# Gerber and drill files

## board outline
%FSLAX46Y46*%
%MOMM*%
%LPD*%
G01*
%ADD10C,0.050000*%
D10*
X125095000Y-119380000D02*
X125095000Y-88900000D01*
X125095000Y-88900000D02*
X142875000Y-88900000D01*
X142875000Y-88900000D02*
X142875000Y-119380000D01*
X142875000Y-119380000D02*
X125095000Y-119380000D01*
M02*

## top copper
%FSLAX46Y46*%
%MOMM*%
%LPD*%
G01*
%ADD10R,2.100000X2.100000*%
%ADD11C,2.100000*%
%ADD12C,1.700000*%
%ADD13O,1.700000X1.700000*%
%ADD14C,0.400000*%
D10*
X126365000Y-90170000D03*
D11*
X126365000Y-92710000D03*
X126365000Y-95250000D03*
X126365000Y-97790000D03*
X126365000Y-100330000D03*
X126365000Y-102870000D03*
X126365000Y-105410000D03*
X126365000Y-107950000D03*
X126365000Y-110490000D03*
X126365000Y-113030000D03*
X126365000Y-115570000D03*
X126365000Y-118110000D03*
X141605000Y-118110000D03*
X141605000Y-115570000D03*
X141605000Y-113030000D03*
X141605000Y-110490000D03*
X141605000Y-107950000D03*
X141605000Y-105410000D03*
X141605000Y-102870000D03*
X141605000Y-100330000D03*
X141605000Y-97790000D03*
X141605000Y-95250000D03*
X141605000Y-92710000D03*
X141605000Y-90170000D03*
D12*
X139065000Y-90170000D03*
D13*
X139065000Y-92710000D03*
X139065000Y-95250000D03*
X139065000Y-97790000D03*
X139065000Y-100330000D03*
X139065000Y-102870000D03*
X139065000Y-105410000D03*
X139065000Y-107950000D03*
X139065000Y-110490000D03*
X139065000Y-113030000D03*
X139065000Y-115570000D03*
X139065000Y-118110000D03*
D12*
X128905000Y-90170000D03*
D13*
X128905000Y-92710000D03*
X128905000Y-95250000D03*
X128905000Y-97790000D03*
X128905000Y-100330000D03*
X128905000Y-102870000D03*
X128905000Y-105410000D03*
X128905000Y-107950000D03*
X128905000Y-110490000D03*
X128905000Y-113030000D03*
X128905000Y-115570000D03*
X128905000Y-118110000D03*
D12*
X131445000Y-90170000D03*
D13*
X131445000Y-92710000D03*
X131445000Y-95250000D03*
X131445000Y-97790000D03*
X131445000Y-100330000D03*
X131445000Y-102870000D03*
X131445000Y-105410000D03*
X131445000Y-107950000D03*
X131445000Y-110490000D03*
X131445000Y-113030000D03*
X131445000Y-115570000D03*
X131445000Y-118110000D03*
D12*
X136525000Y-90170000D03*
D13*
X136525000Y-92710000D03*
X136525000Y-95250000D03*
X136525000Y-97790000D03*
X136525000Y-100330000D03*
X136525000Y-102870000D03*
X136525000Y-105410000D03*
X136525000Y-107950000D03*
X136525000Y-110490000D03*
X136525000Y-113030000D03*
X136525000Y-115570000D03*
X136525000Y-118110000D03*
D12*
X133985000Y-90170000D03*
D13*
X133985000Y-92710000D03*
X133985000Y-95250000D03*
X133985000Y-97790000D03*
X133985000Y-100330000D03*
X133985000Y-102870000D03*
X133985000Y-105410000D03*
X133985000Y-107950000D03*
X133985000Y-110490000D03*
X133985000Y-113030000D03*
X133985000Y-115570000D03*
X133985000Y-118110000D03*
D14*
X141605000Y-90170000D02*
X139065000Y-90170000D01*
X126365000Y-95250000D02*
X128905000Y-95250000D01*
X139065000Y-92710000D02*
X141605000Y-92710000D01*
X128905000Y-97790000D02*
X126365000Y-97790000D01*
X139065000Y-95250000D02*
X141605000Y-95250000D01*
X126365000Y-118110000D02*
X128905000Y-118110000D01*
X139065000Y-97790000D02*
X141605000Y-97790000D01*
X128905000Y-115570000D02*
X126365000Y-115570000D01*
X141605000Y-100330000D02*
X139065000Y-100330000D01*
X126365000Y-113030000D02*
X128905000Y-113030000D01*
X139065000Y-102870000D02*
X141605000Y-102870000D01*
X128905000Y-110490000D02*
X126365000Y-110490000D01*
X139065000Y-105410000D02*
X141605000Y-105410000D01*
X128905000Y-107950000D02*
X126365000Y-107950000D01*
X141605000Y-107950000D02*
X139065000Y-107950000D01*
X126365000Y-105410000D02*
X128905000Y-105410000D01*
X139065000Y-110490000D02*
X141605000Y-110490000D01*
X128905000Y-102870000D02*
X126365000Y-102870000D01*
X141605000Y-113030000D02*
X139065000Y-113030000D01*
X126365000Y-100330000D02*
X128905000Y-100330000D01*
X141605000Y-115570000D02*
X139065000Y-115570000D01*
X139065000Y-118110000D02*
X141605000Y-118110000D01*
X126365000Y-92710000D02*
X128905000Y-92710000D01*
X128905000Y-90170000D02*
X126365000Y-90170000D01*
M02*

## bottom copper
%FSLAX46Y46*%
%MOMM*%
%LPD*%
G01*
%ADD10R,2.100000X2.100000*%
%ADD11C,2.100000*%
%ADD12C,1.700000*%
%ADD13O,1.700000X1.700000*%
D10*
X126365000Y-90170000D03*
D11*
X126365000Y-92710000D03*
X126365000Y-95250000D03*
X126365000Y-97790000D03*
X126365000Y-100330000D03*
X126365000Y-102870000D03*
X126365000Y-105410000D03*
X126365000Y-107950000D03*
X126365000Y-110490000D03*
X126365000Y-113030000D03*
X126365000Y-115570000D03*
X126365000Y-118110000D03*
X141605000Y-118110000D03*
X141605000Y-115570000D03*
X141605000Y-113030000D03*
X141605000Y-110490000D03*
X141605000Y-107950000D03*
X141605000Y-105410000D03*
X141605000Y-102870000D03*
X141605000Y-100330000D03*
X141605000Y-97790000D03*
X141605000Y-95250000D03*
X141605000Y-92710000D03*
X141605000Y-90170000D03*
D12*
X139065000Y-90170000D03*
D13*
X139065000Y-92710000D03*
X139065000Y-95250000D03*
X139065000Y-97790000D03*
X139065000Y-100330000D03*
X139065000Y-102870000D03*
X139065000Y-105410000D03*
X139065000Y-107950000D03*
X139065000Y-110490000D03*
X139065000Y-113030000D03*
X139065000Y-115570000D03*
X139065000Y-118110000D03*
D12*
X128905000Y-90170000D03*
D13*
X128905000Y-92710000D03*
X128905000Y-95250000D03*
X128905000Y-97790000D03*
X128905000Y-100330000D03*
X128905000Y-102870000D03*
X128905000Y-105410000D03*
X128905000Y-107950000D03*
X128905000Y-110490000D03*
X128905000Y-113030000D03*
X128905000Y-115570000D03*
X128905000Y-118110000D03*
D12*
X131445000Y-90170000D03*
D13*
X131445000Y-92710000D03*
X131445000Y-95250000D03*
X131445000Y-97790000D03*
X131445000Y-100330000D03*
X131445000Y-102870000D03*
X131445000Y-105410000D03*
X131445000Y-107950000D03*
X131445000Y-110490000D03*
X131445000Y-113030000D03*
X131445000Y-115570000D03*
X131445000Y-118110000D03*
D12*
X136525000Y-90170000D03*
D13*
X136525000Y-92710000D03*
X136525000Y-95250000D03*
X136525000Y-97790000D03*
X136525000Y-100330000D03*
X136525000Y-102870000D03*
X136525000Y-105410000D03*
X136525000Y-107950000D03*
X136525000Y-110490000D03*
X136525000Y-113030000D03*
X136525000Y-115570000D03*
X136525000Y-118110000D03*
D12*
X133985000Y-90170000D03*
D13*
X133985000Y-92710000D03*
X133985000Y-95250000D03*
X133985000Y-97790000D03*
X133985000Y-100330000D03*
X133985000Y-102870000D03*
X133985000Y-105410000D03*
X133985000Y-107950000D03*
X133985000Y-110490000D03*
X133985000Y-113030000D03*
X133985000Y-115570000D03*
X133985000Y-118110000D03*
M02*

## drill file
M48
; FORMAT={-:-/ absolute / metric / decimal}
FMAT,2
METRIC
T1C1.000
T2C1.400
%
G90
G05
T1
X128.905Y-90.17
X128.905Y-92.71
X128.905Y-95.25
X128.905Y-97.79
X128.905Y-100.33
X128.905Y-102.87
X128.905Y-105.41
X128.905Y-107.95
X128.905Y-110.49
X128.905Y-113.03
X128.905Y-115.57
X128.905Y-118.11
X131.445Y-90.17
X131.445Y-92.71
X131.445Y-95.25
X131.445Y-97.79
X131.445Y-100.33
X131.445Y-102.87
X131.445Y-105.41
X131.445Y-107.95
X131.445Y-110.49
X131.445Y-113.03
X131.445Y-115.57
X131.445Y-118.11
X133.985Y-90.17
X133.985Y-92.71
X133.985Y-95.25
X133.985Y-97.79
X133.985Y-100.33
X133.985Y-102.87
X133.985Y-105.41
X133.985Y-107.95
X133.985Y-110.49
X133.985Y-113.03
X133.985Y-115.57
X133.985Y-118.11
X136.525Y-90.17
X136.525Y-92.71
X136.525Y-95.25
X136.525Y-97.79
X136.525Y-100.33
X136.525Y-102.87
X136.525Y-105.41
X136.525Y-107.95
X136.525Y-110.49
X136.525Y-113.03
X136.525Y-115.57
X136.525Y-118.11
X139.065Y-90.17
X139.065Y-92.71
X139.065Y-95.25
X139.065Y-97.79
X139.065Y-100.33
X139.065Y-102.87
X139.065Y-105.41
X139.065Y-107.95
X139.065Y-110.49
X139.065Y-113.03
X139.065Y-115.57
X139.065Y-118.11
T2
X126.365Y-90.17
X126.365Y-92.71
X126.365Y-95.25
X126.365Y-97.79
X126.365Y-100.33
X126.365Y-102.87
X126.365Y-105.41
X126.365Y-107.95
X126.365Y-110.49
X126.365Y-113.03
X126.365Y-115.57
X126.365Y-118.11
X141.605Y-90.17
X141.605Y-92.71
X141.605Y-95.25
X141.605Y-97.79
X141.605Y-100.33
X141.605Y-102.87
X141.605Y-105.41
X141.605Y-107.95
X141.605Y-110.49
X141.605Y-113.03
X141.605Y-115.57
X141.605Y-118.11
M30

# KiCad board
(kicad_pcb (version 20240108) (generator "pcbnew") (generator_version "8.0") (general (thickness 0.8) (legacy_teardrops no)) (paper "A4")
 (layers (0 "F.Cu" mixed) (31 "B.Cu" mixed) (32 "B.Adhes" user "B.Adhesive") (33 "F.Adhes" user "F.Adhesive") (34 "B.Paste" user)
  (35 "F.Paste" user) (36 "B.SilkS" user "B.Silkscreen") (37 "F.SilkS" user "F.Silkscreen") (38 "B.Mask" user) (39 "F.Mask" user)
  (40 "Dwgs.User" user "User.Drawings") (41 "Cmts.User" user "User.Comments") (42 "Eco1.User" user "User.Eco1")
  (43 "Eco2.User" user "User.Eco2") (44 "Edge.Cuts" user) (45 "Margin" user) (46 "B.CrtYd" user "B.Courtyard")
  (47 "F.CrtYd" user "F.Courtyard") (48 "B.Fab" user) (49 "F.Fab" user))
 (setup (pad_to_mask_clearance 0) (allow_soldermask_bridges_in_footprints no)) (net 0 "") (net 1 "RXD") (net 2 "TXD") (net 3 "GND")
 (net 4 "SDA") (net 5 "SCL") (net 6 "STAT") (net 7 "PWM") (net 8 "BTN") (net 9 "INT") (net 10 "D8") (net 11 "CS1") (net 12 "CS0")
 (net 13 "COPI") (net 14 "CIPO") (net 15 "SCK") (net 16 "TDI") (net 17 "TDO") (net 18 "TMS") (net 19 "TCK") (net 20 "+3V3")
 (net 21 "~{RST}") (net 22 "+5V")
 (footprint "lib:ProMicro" (layer "F.Cu") (at 126.365 90.17)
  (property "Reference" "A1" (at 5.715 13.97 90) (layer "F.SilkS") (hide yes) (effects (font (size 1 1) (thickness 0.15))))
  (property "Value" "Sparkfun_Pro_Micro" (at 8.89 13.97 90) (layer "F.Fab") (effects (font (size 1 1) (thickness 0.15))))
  (pad "1" thru_hole rect (at 0 0) (size 2.1 2.1) (drill 1.4) (layers "*.Cu" "*.Mask") (remove_unused_layers no) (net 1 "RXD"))
  (pad "2" thru_hole circle (at 0 2.54) (size 2.1 2.1) (drill 1.4) (layers "*.Cu" "*.Mask") (remove_unused_layers no) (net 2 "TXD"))
  (pad "3" thru_hole circle (at 0 5.08) (size 2.1 2.1) (drill 1.4) (layers "*.Cu" "*.Mask") (remove_unused_layers no) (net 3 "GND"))
  (pad "4" thru_hole circle (at 0 7.62) (size 2.1 2.1) (drill 1.4) (layers "*.Cu" "*.Mask") (remove_unused_layers no) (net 3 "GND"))
  (pad "5" thru_hole circle (at 0 10.16) (size 2.1 2.1) (drill 1.4) (layers "*.Cu" "*.Mask") (remove_unused_layers no) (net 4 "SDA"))
  (pad "6" thru_hole circle (at 0 12.7) (size 2.1 2.1) (drill 1.4) (layers "*.Cu" "*.Mask") (remove_unused_layers no) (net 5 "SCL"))
  (pad "7" thru_hole circle (at 0 15.24) (size 2.1 2.1) (drill 1.4) (layers "*.Cu" "*.Mask") (remove_unused_layers no) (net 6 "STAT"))
  (pad "8" thru_hole circle (at 0 17.78) (size 2.1 2.1) (drill 1.4) (layers "*.Cu" "*.Mask") (remove_unused_layers no) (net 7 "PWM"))
  (pad "9" thru_hole circle (at 0 20.32) (size 2.1 2.1) (drill 1.4) (layers "*.Cu" "*.Mask") (remove_unused_layers no) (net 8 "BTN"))
  (pad "10" thru_hole circle (at 0 22.86) (size 2.1 2.1) (drill 1.4) (layers "*.Cu" "*.Mask") (remove_unused_layers no) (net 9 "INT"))
  (pad "11" thru_hole circle (at 0 25.4) (size 2.1 2.1) (drill 1.4) (layers "*.Cu" "*.Mask") (remove_unused_layers no) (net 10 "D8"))
  (pad "12" thru_hole circle (at 0 27.94) (size 2.1 2.1) (drill 1.4) (layers "*.Cu" "*.Mask") (remove_unused_layers no) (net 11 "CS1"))
  (pad "13" thru_hole circle (at 15.24 27.94) (size 2.1 2.1) (drill 1.4) (layers "*.Cu" "*.Mask") (remove_unused_layers no) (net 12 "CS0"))
  (pad "14" thru_hole circle (at 15.24 25.4) (size 2.1 2.1) (drill 1.4) (layers "*.Cu" "*.Mask") (remove_unused_layers no) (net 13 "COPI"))
  (pad "15" thru_hole circle (at 15.24 22.86) (size 2.1 2.1) (drill 1.4) (layers "*.Cu" "*.Mask") (remove_unused_layers no) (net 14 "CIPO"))
  (pad "16" thru_hole circle (at 15.24 20.32) (size 2.1 2.1) (drill 1.4) (layers "*.Cu" "*.Mask") (remove_unused_layers no) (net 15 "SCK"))
  (pad "17" thru_hole circle (at 15.24 17.78) (size 2.1 2.1) (drill 1.4) (layers "*.Cu" "*.Mask") (remove_unused_layers no) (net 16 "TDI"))
  (pad "18" thru_hole circle (at 15.24 15.24) (size 2.1 2.1) (drill 1.4) (layers "*.Cu" "*.Mask") (remove_unused_layers no) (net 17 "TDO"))
  (pad "19" thru_hole circle (at 15.24 12.7) (size 2.1 2.1) (drill 1.4) (layers "*.Cu" "*.Mask") (remove_unused_layers no) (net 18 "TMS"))
  (pad "20" thru_hole circle (at 15.24 10.16) (size 2.1 2.1) (drill 1.4) (layers "*.Cu" "*.Mask") (remove_unused_layers no) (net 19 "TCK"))
  (pad "21" thru_hole circle (at 15.24 7.62) (size 2.1 2.1) (drill 1.4) (layers "*.Cu" "*.Mask") (remove_unused_layers no) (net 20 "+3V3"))
  (pad "22" thru_hole circle (at 15.24 5.08) (size 2.1 2.1) (drill 1.4) (layers "*.Cu" "*.Mask") (remove_unused_layers no) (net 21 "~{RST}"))
  (pad "23" thru_hole circle (at 15.24 2.54) (size 2.1 2.1) (drill 1.4) (layers "*.Cu" "*.Mask") (remove_unused_layers no) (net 3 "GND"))
  (pad "24" thru_hole circle (at 15.24 0) (size 2.1 2.1) (drill 1.4) (layers "*.Cu" "*.Mask") (remove_unused_layers no) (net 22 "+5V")))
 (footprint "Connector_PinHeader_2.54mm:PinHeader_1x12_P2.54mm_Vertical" (layer "F.Cu") (at 139.065 90.17)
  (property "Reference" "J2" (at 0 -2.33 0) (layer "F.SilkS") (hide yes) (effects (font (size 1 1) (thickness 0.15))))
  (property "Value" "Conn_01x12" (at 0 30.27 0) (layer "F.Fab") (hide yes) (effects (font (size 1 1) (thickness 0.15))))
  (pad "1" thru_hole circle (at 0 0) (size 1.7 1.7) (drill 1) (layers "*.Cu" "*.Mask") (remove_unused_layers no) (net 22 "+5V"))
  (pad "2" thru_hole oval (at 0 2.54) (size 1.7 1.7) (drill 1) (layers "*.Cu" "*.Mask") (remove_unused_layers no) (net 3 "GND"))
  (pad "3" thru_hole oval (at 0 5.08) (size 1.7 1.7) (drill 1) (layers "*.Cu" "*.Mask") (remove_unused_layers no) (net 21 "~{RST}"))
  (pad "4" thru_hole oval (at 0 7.62) (size 1.7 1.7) (drill 1) (layers "*.Cu" "*.Mask") (remove_unused_layers no) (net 20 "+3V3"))
  (pad "5" thru_hole oval (at 0 10.16) (size 1.7 1.7) (drill 1) (layers "*.Cu" "*.Mask") (remove_unused_layers no) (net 19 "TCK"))
  (pad "6" thru_hole oval (at 0 12.7) (size 1.7 1.7) (drill 1) (layers "*.Cu" "*.Mask") (remove_unused_layers no) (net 18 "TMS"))
  (pad "7" thru_hole oval (at 0 15.24) (size 1.7 1.7) (drill 1) (layers "*.Cu" "*.Mask") (remove_unused_layers no) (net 17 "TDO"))
  (pad "8" thru_hole oval (at 0 17.78) (size 1.7 1.7) (drill 1) (layers "*.Cu" "*.Mask") (remove_unused_layers no) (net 16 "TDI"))
  (pad "9" thru_hole oval (at 0 20.32) (size 1.7 1.7) (drill 1) (layers "*.Cu" "*.Mask") (remove_unused_layers no) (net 15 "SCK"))
  (pad "10" thru_hole oval (at 0 22.86) (size 1.7 1.7) (drill 1) (layers "*.Cu" "*.Mask") (remove_unused_layers no) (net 14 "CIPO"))
  (pad "11" thru_hole oval (at 0 25.4) (size 1.7 1.7) (drill 1) (layers "*.Cu" "*.Mask") (remove_unused_layers no) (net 13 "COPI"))
  (pad "12" thru_hole oval (at 0 27.94) (size 1.7 1.7) (drill 1) (layers "*.Cu" "*.Mask") (remove_unused_layers no) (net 12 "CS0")))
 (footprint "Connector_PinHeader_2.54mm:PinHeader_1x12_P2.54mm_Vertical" (layer "F.Cu") (at 128.905 90.17)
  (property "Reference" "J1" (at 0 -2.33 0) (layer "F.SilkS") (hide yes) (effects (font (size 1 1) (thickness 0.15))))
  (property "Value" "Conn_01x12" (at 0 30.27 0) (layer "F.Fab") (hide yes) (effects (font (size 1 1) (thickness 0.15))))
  (pad "1" thru_hole circle (at 0 0) (size 1.7 1.7) (drill 1) (layers "*.Cu" "*.Mask") (remove_unused_layers no) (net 1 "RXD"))
  (pad "2" thru_hole oval (at 0 2.54) (size 1.7 1.7) (drill 1) (layers "*.Cu" "*.Mask") (remove_unused_layers no) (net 2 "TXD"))
  (pad "3" thru_hole oval (at 0 5.08) (size 1.7 1.7) (drill 1) (layers "*.Cu" "*.Mask") (remove_unused_layers no) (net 3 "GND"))
  (pad "4" thru_hole oval (at 0 7.62) (size 1.7 1.7) (drill 1) (layers "*.Cu" "*.Mask") (remove_unused_layers no) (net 3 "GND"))
  (pad "5" thru_hole oval (at 0 10.16) (size 1.7 1.7) (drill 1) (layers "*.Cu" "*.Mask") (remove_unused_layers no) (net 4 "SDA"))
  (pad "6" thru_hole oval (at 0 12.7) (size 1.7 1.7) (drill 1) (layers "*.Cu" "*.Mask") (remove_unused_layers no) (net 5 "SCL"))
  (pad "7" thru_hole oval (at 0 15.24) (size 1.7 1.7) (drill 1) (layers "*.Cu" "*.Mask") (remove_unused_layers no) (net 6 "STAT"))
  (pad "8" thru_hole oval (at 0 17.78) (size 1.7 1.7) (drill 1) (layers "*.Cu" "*.Mask") (remove_unused_layers no) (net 7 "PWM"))
  (pad "9" thru_hole oval (at 0 20.32) (size 1.7 1.7) (drill 1) (layers "*.Cu" "*.Mask") (remove_unused_layers no) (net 8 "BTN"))
  (pad "10" thru_hole oval (at 0 22.86) (size 1.7 1.7) (drill 1) (layers "*.Cu" "*.Mask") (remove_unused_layers no) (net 9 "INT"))
  (pad "11" thru_hole oval (at 0 25.4) (size 1.7 1.7) (drill 1) (layers "*.Cu" "*.Mask") (remove_unused_layers no) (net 10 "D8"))
  (pad "12" thru_hole oval (at 0 27.94) (size 1.7 1.7) (drill 1) (layers "*.Cu" "*.Mask") (remove_unused_layers no) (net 11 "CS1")))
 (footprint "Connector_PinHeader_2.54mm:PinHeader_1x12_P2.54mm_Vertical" (layer "F.Cu") (at 131.445 90.17)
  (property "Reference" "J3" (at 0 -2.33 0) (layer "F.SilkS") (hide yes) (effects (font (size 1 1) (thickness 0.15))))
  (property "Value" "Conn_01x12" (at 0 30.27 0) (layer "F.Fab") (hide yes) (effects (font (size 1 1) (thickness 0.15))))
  (pad "1" thru_hole circle (at 0 0) (size 1.7 1.7) (drill 1) (layers "*.Cu" "*.Mask") (remove_unused_layers no))
  (pad "2" thru_hole oval (at 0 2.54) (size 1.7 1.7) (drill 1) (layers "*.Cu" "*.Mask") (remove_unused_layers no))
  (pad "3" thru_hole oval (at 0 5.08) (size 1.7 1.7) (drill 1) (layers "*.Cu" "*.Mask") (remove_unused_layers no))
  (pad "4" thru_hole oval (at 0 7.62) (size 1.7 1.7) (drill 1) (layers "*.Cu" "*.Mask") (remove_unused_layers no))
  (pad "5" thru_hole oval (at 0 10.16) (size 1.7 1.7) (drill 1) (layers "*.Cu" "*.Mask") (remove_unused_layers no))
  (pad "6" thru_hole oval (at 0 12.7) (size 1.7 1.7) (drill 1) (layers "*.Cu" "*.Mask") (remove_unused_layers no))
  (pad "7" thru_hole oval (at 0 15.24) (size 1.7 1.7) (drill 1) (layers "*.Cu" "*.Mask") (remove_unused_layers no))
  (pad "8" thru_hole oval (at 0 17.78) (size 1.7 1.7) (drill 1) (layers "*.Cu" "*.Mask") (remove_unused_layers no))
  (pad "9" thru_hole oval (at 0 20.32) (size 1.7 1.7) (drill 1) (layers "*.Cu" "*.Mask") (remove_unused_layers no))
  (pad "10" thru_hole oval (at 0 22.86) (size 1.7 1.7) (drill 1) (layers "*.Cu" "*.Mask") (remove_unused_layers no))
  (pad "11" thru_hole oval (at 0 25.4) (size 1.7 1.7) (drill 1) (layers "*.Cu" "*.Mask") (remove_unused_layers no))
  (pad "12" thru_hole oval (at 0 27.94) (size 1.7 1.7) (drill 1) (layers "*.Cu" "*.Mask") (remove_unused_layers no)))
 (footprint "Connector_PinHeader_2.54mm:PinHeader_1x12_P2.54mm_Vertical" (layer "F.Cu") (at 136.525 90.17)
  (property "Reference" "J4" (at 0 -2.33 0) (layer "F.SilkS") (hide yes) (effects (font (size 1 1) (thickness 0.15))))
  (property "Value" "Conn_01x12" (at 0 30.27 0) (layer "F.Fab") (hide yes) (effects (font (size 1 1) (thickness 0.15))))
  (pad "1" thru_hole circle (at 0 0) (size 1.7 1.7) (drill 1) (layers "*.Cu" "*.Mask") (remove_unused_layers no))
  (pad "2" thru_hole oval (at 0 2.54) (size 1.7 1.7) (drill 1) (layers "*.Cu" "*.Mask") (remove_unused_layers no))
  (pad "3" thru_hole oval (at 0 5.08) (size 1.7 1.7) (drill 1) (layers "*.Cu" "*.Mask") (remove_unused_layers no))
  (pad "4" thru_hole oval (at 0 7.62) (size 1.7 1.7) (drill 1) (layers "*.Cu" "*.Mask") (remove_unused_layers no))
  (pad "5" thru_hole oval (at 0 10.16) (size 1.7 1.7) (drill 1) (layers "*.Cu" "*.Mask") (remove_unused_layers no))
  (pad "6" thru_hole oval (at 0 12.7) (size 1.7 1.7) (drill 1) (layers "*.Cu" "*.Mask") (remove_unused_layers no))
  (pad "7" thru_hole oval (at 0 15.24) (size 1.7 1.7) (drill 1) (layers "*.Cu" "*.Mask") (remove_unused_layers no))
  (pad "8" thru_hole oval (at 0 17.78) (size 1.7 1.7) (drill 1) (layers "*.Cu" "*.Mask") (remove_unused_layers no))
  (pad "9" thru_hole oval (at 0 20.32) (size 1.7 1.7) (drill 1) (layers "*.Cu" "*.Mask") (remove_unused_layers no))
  (pad "10" thru_hole oval (at 0 22.86) (size 1.7 1.7) (drill 1) (layers "*.Cu" "*.Mask") (remove_unused_layers no))
  (pad "11" thru_hole oval (at 0 25.4) (size 1.7 1.7) (drill 1) (layers "*.Cu" "*.Mask") (remove_unused_layers no))
  (pad "12" thru_hole oval (at 0 27.94) (size 1.7 1.7) (drill 1) (layers "*.Cu" "*.Mask") (remove_unused_layers no)))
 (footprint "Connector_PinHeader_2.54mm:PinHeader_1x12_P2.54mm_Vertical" (layer "F.Cu") (at 133.985 90.17)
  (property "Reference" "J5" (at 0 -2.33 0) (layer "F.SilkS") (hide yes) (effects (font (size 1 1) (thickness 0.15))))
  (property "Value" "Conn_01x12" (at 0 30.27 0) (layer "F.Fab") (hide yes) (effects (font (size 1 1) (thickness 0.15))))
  (pad "1" thru_hole circle (at 0 0) (size 1.7 1.7) (drill 1) (layers "*.Cu" "*.Mask") (remove_unused_layers no))
  (pad "2" thru_hole oval (at 0 2.54) (size 1.7 1.7) (drill 1) (layers "*.Cu" "*.Mask") (remove_unused_layers no))
  (pad "3" thru_hole oval (at 0 5.08) (size 1.7 1.7) (drill 1) (layers "*.Cu" "*.Mask") (remove_unused_layers no))
  (pad "4" thru_hole oval (at 0 7.62) (size 1.7 1.7) (drill 1) (layers "*.Cu" "*.Mask") (remove_unused_layers no))
  (pad "5" thru_hole oval (at 0 10.16) (size 1.7 1.7) (drill 1) (layers "*.Cu" "*.Mask") (remove_unused_layers no))
  (pad "6" thru_hole oval (at 0 12.7) (size 1.7 1.7) (drill 1) (layers "*.Cu" "*.Mask") (remove_unused_layers no))
  (pad "7" thru_hole oval (at 0 15.24) (size 1.7 1.7) (drill 1) (layers "*.Cu" "*.Mask") (remove_unused_layers no))
  (pad "8" thru_hole oval (at 0 17.78) (size 1.7 1.7) (drill 1) (layers "*.Cu" "*.Mask") (remove_unused_layers no))
  (pad "9" thru_hole oval (at 0 20.32) (size 1.7 1.7) (drill 1) (layers "*.Cu" "*.Mask") (remove_unused_layers no))
  (pad "10" thru_hole oval (at 0 22.86) (size 1.7 1.7) (drill 1) (layers "*.Cu" "*.Mask") (remove_unused_layers no))
  (pad "11" thru_hole oval (at 0 25.4) (size 1.7 1.7) (drill 1) (layers "*.Cu" "*.Mask") (remove_unused_layers no))
  (pad "12" thru_hole oval (at 0 27.94) (size 1.7 1.7) (drill 1) (layers "*.Cu" "*.Mask") (remove_unused_layers no)))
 (gr_line (start 125.095 119.38) (end 125.095 88.9) (stroke (width 0.05) (type solid)) (layer "Edge.Cuts"))
 (gr_line (start 125.095 88.9) (end 142.875 88.9) (stroke (width 0.05) (type solid)) (layer "Edge.Cuts"))
 (gr_line (start 142.875 88.9) (end 142.875 119.38) (stroke (width 0.05) (type solid)) (layer "Edge.Cuts"))
 (gr_line (start 142.875 119.38) (end 125.095 119.38) (stroke (width 0.05) (type solid)) (layer "Edge.Cuts"))
 (segment (start 141.605 90.17) (end 139.065 90.17) (width 0.4) (layer "F.Cu") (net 22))
 (segment (start 126.365 95.25) (end 128.905 95.25) (width 0.4) (layer "F.Cu") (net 3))
 (segment (start 139.065 92.71) (end 141.605 92.71) (width 0.4) (layer "F.Cu") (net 3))
 (segment (start 128.905 97.79) (end 126.365 97.79) (width 0.4) (layer "F.Cu") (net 3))
 (segment (start 139.065 95.25) (end 141.605 95.25) (width 0.4) (layer "F.Cu") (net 21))
 (segment (start 126.365 118.11) (end 128.905 118.11) (width 0.4) (layer "F.Cu") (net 11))
 (segment (start 139.065 97.79) (end 141.605 97.79) (width 0.4) (layer "F.Cu") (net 20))
 (segment (start 128.905 115.57) (end 126.365 115.57) (width 0.4) (layer "F.Cu") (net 10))
 (segment (start 141.605 100.33) (end 139.065 100.33) (width 0.4) (layer "F.Cu") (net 19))
 (segment (start 126.365 113.03) (end 128.905 113.03) (width 0.4) (layer "F.Cu") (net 9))
 (segment (start 139.065 102.87) (end 141.605 102.87) (width 0.4) (layer "F.Cu") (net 18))
 (segment (start 128.905 110.49) (end 126.365 110.49) (width 0.4) (layer "F.Cu") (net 8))
 (segment (start 139.065 105.41) (end 141.605 105.41) (width 0.4) (layer "F.Cu") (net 17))
 (segment (start 128.905 107.95) (end 126.365 107.95) (width 0.4) (layer "F.Cu") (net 7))
 (segment (start 141.605 107.95) (end 139.065 107.95) (width 0.4) (layer "F.Cu") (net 16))
 (segment (start 126.365 105.41) (end 128.905 105.41) (width 0.4) (layer "F.Cu") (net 6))
 (segment (start 139.065 110.49) (end 141.605 110.49) (width 0.4) (layer "F.Cu") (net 15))
 (segment (start 128.905 102.87) (end 126.365 102.87) (width 0.4) (layer "F.Cu") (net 5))
 (segment (start 141.605 113.03) (end 139.065 113.03) (width 0.4) (layer "F.Cu") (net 14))
 (segment (start 126.365 100.33) (end 128.905 100.33) (width 0.4) (layer "F.Cu") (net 4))
 (segment (start 141.605 115.57) (end 139.065 115.57) (width 0.4) (layer "F.Cu") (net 13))
 (segment (start 139.065 118.11) (end 141.605 118.11) (width 0.4) (layer "F.Cu") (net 12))
 (segment (start 126.365 92.71) (end 128.905 92.71) (width 0.4) (layer "F.Cu") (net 2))
 (segment (start 128.905 90.17) (end 126.365 90.17) (width 0.4) (layer "F.Cu") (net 1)))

